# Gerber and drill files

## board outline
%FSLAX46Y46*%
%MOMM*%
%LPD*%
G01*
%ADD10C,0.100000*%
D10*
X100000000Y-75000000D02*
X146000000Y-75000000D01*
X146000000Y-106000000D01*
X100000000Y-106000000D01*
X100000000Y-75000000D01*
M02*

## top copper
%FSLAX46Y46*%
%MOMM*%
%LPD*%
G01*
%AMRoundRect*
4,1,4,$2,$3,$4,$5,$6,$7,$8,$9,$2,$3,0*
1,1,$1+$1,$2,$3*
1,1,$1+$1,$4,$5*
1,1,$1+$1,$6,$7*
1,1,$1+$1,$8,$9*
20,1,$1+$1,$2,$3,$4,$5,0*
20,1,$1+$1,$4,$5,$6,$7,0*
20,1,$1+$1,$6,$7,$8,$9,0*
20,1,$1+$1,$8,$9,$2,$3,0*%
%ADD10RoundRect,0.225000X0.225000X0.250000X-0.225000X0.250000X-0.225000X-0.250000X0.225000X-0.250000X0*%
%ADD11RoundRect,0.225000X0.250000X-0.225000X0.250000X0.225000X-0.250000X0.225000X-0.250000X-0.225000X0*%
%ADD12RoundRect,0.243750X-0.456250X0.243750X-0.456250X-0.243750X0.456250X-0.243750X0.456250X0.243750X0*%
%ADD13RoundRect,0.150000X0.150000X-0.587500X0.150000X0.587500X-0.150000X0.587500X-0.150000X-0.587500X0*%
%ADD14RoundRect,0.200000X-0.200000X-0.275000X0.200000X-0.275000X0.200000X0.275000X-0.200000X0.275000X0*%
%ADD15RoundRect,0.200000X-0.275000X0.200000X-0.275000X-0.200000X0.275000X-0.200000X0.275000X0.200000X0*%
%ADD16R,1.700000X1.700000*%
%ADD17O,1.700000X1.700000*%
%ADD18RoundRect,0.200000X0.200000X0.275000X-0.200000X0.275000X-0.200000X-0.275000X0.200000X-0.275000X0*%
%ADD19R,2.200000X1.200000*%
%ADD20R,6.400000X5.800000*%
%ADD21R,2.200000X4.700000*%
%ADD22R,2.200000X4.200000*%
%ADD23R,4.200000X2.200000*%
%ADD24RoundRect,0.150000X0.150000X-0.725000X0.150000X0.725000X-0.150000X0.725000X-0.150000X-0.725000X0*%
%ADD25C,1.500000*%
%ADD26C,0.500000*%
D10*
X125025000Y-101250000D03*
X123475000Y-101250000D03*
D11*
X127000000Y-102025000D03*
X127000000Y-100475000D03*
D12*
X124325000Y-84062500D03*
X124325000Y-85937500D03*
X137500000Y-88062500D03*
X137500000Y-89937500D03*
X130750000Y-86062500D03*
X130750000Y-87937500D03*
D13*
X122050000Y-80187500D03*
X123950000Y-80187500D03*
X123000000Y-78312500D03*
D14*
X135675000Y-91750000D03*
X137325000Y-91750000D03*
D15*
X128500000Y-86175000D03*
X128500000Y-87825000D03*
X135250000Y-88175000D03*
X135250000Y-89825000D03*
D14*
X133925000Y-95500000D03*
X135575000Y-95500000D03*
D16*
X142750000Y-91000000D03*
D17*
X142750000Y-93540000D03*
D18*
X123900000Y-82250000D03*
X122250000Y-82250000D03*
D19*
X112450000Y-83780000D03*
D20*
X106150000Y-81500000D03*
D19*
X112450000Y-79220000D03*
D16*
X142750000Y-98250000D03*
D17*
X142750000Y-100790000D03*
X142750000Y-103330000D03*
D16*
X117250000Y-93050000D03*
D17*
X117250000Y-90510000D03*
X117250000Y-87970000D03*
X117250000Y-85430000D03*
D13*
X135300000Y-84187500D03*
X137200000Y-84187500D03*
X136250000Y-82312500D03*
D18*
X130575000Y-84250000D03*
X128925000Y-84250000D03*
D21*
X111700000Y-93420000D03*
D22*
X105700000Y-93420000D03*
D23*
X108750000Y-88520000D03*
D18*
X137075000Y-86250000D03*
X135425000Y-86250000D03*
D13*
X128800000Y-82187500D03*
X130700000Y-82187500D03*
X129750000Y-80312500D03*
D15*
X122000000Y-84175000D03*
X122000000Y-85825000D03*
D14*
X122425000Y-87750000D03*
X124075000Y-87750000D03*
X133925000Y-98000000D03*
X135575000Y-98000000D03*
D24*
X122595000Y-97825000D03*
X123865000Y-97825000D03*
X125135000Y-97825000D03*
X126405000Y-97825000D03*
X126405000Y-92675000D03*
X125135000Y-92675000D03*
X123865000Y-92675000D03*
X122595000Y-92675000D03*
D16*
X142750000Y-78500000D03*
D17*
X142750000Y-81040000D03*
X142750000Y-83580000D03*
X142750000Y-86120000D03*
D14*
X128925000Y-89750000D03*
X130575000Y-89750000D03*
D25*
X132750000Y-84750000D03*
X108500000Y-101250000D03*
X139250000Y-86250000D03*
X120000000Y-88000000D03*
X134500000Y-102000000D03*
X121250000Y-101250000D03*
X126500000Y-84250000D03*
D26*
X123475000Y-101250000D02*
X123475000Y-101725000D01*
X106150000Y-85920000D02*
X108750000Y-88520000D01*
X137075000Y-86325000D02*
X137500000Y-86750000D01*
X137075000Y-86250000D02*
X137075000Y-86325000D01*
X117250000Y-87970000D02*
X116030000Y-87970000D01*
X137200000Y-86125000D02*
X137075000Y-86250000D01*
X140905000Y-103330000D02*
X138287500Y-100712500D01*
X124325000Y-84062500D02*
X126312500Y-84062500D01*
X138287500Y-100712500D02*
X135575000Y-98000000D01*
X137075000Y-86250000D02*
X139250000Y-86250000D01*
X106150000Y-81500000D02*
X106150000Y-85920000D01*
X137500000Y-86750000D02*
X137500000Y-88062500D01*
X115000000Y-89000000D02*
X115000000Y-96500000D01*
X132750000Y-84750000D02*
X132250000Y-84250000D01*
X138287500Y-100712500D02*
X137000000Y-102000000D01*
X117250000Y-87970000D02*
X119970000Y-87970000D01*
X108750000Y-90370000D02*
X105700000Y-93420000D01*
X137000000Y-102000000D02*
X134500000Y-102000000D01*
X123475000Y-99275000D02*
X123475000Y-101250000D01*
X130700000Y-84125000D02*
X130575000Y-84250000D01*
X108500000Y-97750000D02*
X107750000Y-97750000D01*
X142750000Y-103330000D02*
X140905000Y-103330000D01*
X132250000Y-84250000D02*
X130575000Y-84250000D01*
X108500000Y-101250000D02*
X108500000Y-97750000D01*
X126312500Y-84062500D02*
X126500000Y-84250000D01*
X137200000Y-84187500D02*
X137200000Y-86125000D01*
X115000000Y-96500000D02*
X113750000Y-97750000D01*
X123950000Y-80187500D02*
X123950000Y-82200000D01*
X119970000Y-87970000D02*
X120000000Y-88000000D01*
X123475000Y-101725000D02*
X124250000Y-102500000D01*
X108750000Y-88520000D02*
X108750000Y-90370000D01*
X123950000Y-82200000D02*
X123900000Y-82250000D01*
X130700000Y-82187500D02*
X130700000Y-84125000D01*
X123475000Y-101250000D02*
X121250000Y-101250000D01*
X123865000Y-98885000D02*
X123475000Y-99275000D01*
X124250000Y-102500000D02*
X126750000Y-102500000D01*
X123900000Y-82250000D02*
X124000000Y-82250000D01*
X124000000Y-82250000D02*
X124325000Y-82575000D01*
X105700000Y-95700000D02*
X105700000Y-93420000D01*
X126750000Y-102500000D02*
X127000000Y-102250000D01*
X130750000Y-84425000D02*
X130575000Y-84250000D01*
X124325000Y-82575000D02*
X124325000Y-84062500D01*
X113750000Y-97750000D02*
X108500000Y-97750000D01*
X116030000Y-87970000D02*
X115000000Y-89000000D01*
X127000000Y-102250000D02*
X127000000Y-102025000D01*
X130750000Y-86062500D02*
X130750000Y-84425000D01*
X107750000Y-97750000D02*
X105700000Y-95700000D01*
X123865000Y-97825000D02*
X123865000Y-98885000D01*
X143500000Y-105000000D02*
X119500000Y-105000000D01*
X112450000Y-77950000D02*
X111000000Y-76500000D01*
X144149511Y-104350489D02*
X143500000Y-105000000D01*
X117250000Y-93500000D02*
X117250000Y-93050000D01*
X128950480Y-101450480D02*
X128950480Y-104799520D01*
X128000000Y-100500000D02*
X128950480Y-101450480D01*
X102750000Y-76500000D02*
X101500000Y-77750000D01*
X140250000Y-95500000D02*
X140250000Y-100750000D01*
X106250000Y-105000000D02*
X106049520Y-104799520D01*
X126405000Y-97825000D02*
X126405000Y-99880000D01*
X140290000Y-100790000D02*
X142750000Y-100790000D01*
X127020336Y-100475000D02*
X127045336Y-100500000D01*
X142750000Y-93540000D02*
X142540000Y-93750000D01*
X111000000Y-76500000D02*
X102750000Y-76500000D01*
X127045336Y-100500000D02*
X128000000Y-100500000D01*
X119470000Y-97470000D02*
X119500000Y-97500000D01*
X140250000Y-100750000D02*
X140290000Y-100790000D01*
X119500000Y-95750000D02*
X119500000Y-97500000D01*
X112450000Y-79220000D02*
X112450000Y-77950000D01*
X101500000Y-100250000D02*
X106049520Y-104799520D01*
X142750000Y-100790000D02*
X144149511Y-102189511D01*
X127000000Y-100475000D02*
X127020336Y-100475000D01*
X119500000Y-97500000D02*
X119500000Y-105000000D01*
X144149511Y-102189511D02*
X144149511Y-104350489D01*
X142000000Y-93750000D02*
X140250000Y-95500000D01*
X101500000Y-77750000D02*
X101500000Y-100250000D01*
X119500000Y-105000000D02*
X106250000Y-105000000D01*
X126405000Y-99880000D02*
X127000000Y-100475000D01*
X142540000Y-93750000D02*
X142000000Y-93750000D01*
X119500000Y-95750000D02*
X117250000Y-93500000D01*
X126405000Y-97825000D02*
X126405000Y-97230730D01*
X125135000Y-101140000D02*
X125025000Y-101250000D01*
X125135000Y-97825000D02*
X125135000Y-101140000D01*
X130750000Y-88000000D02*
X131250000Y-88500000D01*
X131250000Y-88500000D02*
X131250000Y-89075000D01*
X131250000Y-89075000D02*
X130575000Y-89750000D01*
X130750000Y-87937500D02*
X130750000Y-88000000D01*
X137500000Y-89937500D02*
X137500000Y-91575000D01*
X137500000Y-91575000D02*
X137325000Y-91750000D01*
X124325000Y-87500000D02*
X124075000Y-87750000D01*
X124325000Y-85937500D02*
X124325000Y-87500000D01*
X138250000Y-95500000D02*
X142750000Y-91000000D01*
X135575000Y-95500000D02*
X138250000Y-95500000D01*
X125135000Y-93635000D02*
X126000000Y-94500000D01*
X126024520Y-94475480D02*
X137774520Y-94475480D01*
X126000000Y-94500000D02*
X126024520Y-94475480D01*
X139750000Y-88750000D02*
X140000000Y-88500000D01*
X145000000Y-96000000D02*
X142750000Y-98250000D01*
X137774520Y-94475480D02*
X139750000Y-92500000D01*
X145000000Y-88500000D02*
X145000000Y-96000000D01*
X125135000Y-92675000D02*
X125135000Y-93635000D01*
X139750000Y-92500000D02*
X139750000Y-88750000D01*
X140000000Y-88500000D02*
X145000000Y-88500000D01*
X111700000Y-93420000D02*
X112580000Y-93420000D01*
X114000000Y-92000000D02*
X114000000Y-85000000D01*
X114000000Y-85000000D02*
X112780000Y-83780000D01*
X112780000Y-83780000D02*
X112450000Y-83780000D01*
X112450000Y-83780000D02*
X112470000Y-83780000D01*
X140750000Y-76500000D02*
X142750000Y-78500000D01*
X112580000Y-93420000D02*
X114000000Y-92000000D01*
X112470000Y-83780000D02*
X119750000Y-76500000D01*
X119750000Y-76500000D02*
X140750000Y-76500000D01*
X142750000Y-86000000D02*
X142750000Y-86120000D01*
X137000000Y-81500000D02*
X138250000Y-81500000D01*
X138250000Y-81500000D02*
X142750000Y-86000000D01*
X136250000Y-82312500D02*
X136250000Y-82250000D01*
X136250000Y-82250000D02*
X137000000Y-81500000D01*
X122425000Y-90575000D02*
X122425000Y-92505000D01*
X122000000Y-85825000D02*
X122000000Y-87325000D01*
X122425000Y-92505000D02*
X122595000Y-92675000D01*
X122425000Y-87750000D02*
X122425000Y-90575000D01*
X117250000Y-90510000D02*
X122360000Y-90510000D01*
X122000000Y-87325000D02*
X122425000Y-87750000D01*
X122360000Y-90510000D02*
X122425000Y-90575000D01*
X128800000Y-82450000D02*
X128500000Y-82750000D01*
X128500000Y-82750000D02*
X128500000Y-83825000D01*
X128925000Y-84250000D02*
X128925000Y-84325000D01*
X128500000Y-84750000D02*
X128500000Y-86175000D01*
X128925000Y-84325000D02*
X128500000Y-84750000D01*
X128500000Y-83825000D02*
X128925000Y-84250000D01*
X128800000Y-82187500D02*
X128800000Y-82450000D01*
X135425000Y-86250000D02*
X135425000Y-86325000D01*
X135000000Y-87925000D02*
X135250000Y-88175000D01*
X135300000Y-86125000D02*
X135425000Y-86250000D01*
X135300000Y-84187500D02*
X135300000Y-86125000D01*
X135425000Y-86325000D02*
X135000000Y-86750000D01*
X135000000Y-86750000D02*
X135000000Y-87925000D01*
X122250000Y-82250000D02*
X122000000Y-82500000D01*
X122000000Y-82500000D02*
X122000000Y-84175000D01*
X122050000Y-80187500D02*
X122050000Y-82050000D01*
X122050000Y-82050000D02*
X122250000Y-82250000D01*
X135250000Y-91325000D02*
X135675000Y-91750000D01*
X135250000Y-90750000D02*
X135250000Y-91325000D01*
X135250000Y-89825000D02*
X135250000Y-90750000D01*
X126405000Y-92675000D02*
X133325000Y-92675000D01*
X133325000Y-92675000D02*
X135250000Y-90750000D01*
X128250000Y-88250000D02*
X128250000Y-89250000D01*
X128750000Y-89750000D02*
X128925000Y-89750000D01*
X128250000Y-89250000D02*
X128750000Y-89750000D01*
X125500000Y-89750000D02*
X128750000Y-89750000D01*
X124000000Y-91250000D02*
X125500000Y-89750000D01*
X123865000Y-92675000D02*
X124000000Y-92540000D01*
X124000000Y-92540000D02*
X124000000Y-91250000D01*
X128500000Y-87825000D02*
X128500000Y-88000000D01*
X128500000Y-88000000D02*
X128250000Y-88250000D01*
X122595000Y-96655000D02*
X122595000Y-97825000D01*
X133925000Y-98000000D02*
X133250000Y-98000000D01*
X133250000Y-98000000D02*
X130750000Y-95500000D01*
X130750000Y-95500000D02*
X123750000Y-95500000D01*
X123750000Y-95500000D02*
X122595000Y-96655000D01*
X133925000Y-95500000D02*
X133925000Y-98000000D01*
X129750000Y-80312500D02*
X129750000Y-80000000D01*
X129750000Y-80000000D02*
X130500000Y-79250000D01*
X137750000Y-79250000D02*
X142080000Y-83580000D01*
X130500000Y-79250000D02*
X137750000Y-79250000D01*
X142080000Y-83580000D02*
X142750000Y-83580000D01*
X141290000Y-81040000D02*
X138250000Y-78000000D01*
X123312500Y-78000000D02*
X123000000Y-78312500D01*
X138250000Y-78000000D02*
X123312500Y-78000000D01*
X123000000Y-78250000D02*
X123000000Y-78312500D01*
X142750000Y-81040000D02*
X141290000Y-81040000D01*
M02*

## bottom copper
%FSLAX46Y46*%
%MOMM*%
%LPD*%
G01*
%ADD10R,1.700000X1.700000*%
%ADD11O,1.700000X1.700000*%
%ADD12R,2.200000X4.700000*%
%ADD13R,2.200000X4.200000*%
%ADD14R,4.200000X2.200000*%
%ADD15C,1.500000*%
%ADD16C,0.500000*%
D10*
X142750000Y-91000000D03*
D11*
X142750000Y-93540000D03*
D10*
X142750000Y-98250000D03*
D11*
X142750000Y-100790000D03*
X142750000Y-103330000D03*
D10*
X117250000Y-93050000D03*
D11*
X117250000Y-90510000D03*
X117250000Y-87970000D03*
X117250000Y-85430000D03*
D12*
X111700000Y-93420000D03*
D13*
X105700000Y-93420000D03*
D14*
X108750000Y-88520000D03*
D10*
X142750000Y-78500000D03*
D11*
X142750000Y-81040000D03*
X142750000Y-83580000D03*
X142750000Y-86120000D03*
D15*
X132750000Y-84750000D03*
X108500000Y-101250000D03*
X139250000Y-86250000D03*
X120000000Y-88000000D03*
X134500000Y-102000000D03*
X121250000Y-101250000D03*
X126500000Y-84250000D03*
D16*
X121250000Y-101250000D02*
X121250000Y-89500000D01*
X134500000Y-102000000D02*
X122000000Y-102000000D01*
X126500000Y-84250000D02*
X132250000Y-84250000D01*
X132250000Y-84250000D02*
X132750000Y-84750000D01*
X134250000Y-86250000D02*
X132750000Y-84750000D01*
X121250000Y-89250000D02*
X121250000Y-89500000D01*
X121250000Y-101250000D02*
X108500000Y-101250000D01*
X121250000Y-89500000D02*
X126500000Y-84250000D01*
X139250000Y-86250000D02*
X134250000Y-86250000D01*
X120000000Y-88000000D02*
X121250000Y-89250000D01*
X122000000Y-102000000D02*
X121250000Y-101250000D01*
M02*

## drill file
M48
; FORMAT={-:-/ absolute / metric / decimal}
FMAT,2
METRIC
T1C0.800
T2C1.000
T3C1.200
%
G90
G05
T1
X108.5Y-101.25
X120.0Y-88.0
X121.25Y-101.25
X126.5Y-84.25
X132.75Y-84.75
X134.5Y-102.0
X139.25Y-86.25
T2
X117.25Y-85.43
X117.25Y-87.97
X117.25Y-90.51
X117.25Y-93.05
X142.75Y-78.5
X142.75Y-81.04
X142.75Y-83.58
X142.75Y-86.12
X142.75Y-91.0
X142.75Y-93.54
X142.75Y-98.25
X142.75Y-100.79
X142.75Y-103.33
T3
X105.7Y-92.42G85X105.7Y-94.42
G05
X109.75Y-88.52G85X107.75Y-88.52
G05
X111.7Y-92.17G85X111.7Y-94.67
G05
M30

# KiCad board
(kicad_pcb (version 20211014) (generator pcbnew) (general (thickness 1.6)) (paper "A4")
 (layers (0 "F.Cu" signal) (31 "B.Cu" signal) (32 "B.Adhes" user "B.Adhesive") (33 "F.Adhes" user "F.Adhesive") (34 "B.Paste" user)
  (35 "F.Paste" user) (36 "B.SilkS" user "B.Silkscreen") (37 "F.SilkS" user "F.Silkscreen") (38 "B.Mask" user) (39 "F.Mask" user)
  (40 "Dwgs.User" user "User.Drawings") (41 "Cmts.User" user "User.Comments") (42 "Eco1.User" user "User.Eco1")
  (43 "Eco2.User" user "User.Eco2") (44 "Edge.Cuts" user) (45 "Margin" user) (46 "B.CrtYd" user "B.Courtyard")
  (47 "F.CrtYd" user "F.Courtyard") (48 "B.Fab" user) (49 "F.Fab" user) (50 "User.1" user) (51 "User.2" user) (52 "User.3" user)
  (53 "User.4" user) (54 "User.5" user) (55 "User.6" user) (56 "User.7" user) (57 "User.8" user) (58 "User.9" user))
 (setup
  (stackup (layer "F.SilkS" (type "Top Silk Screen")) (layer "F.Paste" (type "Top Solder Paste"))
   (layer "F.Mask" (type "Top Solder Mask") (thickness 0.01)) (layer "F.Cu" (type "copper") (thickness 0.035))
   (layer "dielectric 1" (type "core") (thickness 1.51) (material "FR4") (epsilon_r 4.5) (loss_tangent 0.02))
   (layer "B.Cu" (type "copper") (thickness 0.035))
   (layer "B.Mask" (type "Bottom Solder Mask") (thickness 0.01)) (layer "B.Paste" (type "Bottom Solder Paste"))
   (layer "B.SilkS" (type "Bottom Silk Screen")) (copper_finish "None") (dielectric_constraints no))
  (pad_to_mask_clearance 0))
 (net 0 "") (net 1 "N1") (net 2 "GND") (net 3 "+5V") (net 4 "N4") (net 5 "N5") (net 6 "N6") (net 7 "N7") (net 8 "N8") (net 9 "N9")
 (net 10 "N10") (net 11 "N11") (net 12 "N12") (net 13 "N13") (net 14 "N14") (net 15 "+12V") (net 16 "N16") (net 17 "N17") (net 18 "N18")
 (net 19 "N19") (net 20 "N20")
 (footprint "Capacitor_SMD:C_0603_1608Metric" (layer "F.Cu") (at 124.25 101.25 180)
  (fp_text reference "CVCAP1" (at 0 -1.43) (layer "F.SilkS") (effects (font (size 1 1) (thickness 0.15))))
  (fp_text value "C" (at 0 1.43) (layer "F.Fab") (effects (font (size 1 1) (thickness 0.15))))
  (pad "1" smd roundrect (at -0.775 0 180) (size 0.9 0.95) (layers "F.Cu" "F.Paste" "F.Mask") (roundrect_rratio 0.25) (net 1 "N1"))
  (pad "2" smd roundrect (at 0.775 0 180) (size 0.9 0.95) (layers "F.Cu" "F.Paste" "F.Mask") (roundrect_rratio 0.25) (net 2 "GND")))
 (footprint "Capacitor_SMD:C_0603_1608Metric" (layer "F.Cu") (at 127 101.25 90)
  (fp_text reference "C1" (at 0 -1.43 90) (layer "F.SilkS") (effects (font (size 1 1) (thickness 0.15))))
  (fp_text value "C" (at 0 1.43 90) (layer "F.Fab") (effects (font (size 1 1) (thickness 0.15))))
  (pad "1" smd roundrect (at -0.775 0 90) (size 0.9 0.95) (layers "F.Cu" "F.Paste" "F.Mask") (roundrect_rratio 0.25) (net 2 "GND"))
  (pad "2" smd roundrect (at 0.775 0 90) (size 0.9 0.95) (layers "F.Cu" "F.Paste" "F.Mask") (roundrect_rratio 0.25) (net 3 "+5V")))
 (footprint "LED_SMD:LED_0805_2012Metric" (layer "F.Cu") (at 124.325 85 -90)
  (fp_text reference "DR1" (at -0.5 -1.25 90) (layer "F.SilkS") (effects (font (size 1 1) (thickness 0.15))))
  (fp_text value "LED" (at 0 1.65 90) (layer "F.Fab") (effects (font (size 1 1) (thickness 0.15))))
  (pad "1" smd roundrect (at -0.9375 0 270) (size 0.975 1.4) (layers "F.Cu" "F.Paste" "F.Mask") (roundrect_rratio 0.25) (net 2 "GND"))
  (pad "2" smd roundrect (at 0.9375 0 270) (size 0.975 1.4) (layers "F.Cu" "F.Paste" "F.Mask") (roundrect_rratio 0.25) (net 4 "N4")))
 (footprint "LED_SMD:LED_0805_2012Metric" (layer "F.Cu") (at 137.5 89 -90)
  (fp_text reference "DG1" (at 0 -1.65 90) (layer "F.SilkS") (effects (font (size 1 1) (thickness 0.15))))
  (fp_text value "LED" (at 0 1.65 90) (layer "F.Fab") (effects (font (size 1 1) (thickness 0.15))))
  (pad "1" smd roundrect (at -0.9375 0 270) (size 0.975 1.4) (layers "F.Cu" "F.Paste" "F.Mask") (roundrect_rratio 0.25) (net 2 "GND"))
  (pad "2" smd roundrect (at 0.9375 0 270) (size 0.975 1.4) (layers "F.Cu" "F.Paste" "F.Mask") (roundrect_rratio 0.25) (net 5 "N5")))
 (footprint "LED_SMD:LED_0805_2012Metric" (layer "F.Cu") (at 130.75 87 -90)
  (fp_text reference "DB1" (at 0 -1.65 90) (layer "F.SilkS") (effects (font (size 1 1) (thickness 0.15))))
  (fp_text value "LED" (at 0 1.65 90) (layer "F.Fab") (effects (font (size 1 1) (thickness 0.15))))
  (pad "1" smd roundrect (at -0.9375 0 270) (size 0.975 1.4) (layers "F.Cu" "F.Paste" "F.Mask") (roundrect_rratio 0.25) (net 2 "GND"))
  (pad "2" smd roundrect (at 0.9375 0 270) (size 0.975 1.4) (layers "F.Cu" "F.Paste" "F.Mask") (roundrect_rratio 0.25) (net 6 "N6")))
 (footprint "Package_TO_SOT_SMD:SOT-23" (layer "F.Cu") (at 123 79.25 90)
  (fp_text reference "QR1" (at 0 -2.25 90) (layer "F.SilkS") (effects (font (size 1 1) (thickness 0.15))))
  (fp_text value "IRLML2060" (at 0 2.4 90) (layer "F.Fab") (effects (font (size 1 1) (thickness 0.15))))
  (pad "1" smd roundrect (at -0.9375 -0.95 90) (size 1.475 0.6) (layers "F.Cu" "F.Paste" "F.Mask") (roundrect_rratio 0.25) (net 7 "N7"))
  (pad "2" smd roundrect (at -0.9375 0.95 90) (size 1.475 0.6) (layers "F.Cu" "F.Paste" "F.Mask") (roundrect_rratio 0.25) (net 2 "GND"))
  (pad "3" smd roundrect (at 0.9375 0 90) (size 1.475 0.6) (layers "F.Cu" "F.Paste" "F.Mask") (roundrect_rratio 0.25) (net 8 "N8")))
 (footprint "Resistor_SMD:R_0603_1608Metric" (layer "F.Cu") (at 136.5 91.75)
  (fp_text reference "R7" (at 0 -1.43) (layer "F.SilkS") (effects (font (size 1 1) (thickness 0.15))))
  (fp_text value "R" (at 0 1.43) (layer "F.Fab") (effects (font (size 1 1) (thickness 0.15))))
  (pad "1" smd roundrect (at -0.825 0) (size 0.8 0.95) (layers "F.Cu" "F.Paste" "F.Mask") (roundrect_rratio 0.25) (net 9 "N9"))
  (pad "2" smd roundrect (at 0.825 0) (size 0.8 0.95) (layers "F.Cu" "F.Paste" "F.Mask") (roundrect_rratio 0.25) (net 5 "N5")))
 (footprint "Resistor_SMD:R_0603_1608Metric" (layer "F.Cu") (at 128.5 87 -90)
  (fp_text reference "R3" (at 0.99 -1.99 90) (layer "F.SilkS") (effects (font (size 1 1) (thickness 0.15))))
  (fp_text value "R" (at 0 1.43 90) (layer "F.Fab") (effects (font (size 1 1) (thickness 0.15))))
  (pad "1" smd roundrect (at -0.825 0 270) (size 0.8 0.95) (layers "F.Cu" "F.Paste" "F.Mask") (roundrect_rratio 0.25) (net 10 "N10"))
  (pad "2" smd roundrect (at 0.825 0 270) (size 0.8 0.95) (layers "F.Cu" "F.Paste" "F.Mask") (roundrect_rratio 0.25) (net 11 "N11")))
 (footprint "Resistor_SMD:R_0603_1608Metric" (layer "F.Cu") (at 135.25 89 -90)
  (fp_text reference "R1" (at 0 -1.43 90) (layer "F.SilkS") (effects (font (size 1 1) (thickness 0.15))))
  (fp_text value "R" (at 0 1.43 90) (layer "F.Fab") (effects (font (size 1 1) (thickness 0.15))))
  (pad "1" smd roundrect (at -0.825 0 270) (size 0.8 0.95) (layers "F.Cu" "F.Paste" "F.Mask") (roundrect_rratio 0.25) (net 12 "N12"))
  (pad "2" smd roundrect (at 0.825 0 270) (size 0.8 0.95) (layers "F.Cu" "F.Paste" "F.Mask") (roundrect_rratio 0.25) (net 9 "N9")))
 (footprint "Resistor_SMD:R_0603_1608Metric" (layer "F.Cu") (at 134.75 95.5)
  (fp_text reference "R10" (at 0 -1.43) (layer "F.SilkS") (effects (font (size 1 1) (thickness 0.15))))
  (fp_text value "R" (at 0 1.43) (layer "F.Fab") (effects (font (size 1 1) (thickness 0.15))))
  (pad "1" smd roundrect (at -0.825 0) (size 0.8 0.95) (layers "F.Cu" "F.Paste" "F.Mask") (roundrect_rratio 0.25) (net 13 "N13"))
  (pad "2" smd roundrect (at 0.825 0) (size 0.8 0.95) (layers "F.Cu" "F.Paste" "F.Mask") (roundrect_rratio 0.25) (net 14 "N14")))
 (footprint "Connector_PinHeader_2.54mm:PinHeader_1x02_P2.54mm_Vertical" (layer "F.Cu") (at 142.75 91)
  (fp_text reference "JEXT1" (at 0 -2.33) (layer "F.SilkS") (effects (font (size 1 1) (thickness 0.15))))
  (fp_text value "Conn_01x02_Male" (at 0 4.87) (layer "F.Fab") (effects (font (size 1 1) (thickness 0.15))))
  (pad "1" thru_hole rect (at 0 0) (size 1.7 1.7) (drill 1) (layers *.Cu *.Mask) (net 14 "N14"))
  (pad "2" thru_hole oval (at 0 2.54) (size 1.7 1.7) (drill 1) (layers *.Cu *.Mask) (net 3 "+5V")))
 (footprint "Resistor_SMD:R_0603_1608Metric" (layer "F.Cu") (at 123.075 82.25 180)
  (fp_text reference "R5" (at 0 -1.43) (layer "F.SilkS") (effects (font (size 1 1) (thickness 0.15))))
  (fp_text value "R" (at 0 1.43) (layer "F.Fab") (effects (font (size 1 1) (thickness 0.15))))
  (pad "1" smd roundrect (at -0.825 0 180) (size 0.8 0.95) (layers "F.Cu" "F.Paste" "F.Mask") (roundrect_rratio 0.25) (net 2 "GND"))
  (pad "2" smd roundrect (at 0.825 0 180) (size 0.8 0.95) (layers "F.Cu" "F.Paste" "F.Mask") (roundrect_rratio 0.25) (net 7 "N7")))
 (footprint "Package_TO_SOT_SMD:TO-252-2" (layer "F.Cu") (at 108.25 81.5 180)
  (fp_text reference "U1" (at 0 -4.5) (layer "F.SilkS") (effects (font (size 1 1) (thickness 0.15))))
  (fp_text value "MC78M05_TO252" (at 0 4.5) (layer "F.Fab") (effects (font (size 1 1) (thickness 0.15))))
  (pad "" smd rect (at 3.775 1.525 180) (size 3.05 2.75) (layers "F.Paste"))
  (pad "" smd rect (at 0.425 -1.525 180) (size 3.05 2.75) (layers "F.Paste"))
  (pad "" smd rect (at 0.425 1.525 180) (size 3.05 2.75) (layers "F.Paste"))
  (pad "" smd rect (at 3.775 -1.525 180) (size 3.05 2.75) (layers "F.Paste"))
  (pad "1" smd rect (at -4.2 -2.28 180) (size 2.2 1.2) (layers "F.Cu" "F.Paste" "F.Mask") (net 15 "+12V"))
  (pad "2" smd rect (at 2.1 0 180) (size 6.4 5.8) (layers "F.Cu" "F.Mask") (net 2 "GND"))
  (pad "3" smd rect (at -4.2 2.28 180) (size 2.2 1.2) (layers "F.Cu" "F.Paste" "F.Mask") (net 3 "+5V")))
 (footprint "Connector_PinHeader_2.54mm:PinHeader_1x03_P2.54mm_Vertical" (layer "F.Cu") (at 142.75 98.25)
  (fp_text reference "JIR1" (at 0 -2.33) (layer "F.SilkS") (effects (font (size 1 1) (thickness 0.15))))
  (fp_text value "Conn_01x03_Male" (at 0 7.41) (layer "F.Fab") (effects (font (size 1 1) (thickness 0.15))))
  (pad "1" thru_hole rect (at 0 0) (size 1.7 1.7) (drill 1) (layers *.Cu *.Mask) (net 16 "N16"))
  (pad "2" thru_hole oval (at 0 2.54) (size 1.7 1.7) (drill 1) (layers *.Cu *.Mask) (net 3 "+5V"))
  (pad "3" thru_hole oval (at 0 5.08) (size 1.7 1.7) (drill 1) (layers *.Cu *.Mask) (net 2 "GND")))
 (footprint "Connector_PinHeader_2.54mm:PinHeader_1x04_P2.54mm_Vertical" (layer "F.Cu") (at 117.25 93.05 180)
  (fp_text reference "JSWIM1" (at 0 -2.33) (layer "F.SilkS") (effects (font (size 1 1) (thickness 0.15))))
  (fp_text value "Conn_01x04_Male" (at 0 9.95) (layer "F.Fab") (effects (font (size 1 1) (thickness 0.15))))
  (pad "1" thru_hole rect (at 0 0 180) (size 1.7 1.7) (drill 1) (layers *.Cu *.Mask) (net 3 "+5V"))
  (pad "2" thru_hole oval (at 0 2.54 180) (size 1.7 1.7) (drill 1) (layers *.Cu *.Mask) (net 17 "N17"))
  (pad "3" thru_hole oval (at 0 5.08 180) (size 1.7 1.7) (drill 1) (layers *.Cu *.Mask) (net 2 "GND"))
  (pad "4" thru_hole oval (at 0 7.62 180) (size 1.7 1.7) (drill 1) (layers *.Cu *.Mask) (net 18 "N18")))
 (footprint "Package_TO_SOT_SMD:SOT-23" (layer "F.Cu") (at 136.25 83.25 90)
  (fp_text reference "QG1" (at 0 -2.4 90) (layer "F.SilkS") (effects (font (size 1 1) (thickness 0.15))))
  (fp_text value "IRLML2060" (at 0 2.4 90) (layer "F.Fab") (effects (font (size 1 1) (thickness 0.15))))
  (pad "1" smd roundrect (at -0.9375 -0.95 90) (size 1.475 0.6) (layers "F.Cu" "F.Paste" "F.Mask") (roundrect_rratio 0.25) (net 12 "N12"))
  (pad "2" smd roundrect (at -0.9375 0.95 90) (size 1.475 0.6) (layers "F.Cu" "F.Paste" "F.Mask") (roundrect_rratio 0.25) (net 2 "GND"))
  (pad "3" smd roundrect (at 0.9375 0 90) (size 1.475 0.6) (layers "F.Cu" "F.Paste" "F.Mask") (roundrect_rratio 0.25) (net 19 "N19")))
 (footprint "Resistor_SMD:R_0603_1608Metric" (layer "F.Cu") (at 129.75 84.25 180)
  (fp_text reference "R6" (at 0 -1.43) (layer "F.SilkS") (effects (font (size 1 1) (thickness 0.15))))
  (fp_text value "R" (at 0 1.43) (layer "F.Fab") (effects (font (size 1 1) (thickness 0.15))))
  (pad "1" smd roundrect (at -0.825 0 180) (size 0.8 0.95) (layers "F.Cu" "F.Paste" "F.Mask") (roundrect_rratio 0.25) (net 2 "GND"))
  (pad "2" smd roundrect (at 0.825 0 180) (size 0.8 0.95) (layers "F.Cu" "F.Paste" "F.Mask") (roundrect_rratio 0.25) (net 10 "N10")))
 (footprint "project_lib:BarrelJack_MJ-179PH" (layer "F.Cu") (at 112.5 94 -90)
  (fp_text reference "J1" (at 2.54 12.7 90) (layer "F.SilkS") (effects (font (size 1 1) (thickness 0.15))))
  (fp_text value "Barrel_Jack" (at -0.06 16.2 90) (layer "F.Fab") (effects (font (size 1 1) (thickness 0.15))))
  (pad "1" thru_hole rect (at -0.58 0.8 270) (size 4.7 2.2) (drill oval 3.7 1.2) (layers *.Cu *.Mask) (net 15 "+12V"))
  (pad "2" thru_hole rect (at -0.58 6.8 270) (size 4.2 2.2) (drill oval 3.2 1.2) (layers *.Cu *.Mask) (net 2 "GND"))
  (pad "3" thru_hole rect (at -5.48 3.75 270) (size 2.2 4.2) (drill oval 1.2 3.2) (layers *.Cu *.Mask) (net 2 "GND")))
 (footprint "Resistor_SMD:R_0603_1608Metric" (layer "F.Cu") (at 136.25 86.25 180)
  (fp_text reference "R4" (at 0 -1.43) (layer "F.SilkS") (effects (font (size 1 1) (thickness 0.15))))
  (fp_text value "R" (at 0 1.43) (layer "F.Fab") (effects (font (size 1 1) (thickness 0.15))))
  (pad "1" smd roundrect (at -0.825 0 180) (size 0.8 0.95) (layers "F.Cu" "F.Paste" "F.Mask") (roundrect_rratio 0.25) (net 2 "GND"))
  (pad "2" smd roundrect (at 0.825 0 180) (size 0.8 0.95) (layers "F.Cu" "F.Paste" "F.Mask") (roundrect_rratio 0.25) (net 12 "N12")))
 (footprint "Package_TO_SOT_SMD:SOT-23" (layer "F.Cu") (at 129.75 81.25 90)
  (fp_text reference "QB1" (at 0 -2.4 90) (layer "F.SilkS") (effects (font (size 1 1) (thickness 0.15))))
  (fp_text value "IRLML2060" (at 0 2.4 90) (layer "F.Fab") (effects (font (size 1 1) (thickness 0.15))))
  (pad "1" smd roundrect (at -0.9375 -0.95 90) (size 1.475 0.6) (layers "F.Cu" "F.Paste" "F.Mask") (roundrect_rratio 0.25) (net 10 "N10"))
  (pad "2" smd roundrect (at -0.9375 0.95 90) (size 1.475 0.6) (layers "F.Cu" "F.Paste" "F.Mask") (roundrect_rratio 0.25) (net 2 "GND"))
  (pad "3" smd roundrect (at 0.9375 0 90) (size 1.475 0.6) (layers "F.Cu" "F.Paste" "F.Mask") (roundrect_rratio 0.25) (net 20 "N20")))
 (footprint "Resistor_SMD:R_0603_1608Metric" (layer "F.Cu") (at 122 85 -90)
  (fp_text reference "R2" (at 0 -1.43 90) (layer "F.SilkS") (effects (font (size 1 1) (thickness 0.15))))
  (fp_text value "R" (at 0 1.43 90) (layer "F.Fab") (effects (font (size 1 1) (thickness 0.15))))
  (pad "1" smd roundrect (at -0.825 0 270) (size 0.8 0.95) (layers "F.Cu" "F.Paste" "F.Mask") (roundrect_rratio 0.25) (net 7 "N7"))
  (pad "2" smd roundrect (at 0.825 0 270) (size 0.8 0.95) (layers "F.Cu" "F.Paste" "F.Mask") (roundrect_rratio 0.25) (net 17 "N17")))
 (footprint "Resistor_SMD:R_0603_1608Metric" (layer "F.Cu") (at 123.25 87.75)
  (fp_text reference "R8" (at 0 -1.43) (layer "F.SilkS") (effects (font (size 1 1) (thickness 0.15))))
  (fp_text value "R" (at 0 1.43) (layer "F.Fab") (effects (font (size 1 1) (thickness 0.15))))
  (pad "1" smd roundrect (at -0.825 0) (size 0.8 0.95) (layers "F.Cu" "F.Paste" "F.Mask") (roundrect_rratio 0.25) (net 17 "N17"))
  (pad "2" smd roundrect (at 0.825 0) (size 0.8 0.95) (layers "F.Cu" "F.Paste" "F.Mask") (roundrect_rratio 0.25) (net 4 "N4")))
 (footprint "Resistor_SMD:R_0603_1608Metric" (layer "F.Cu") (at 134.75 98)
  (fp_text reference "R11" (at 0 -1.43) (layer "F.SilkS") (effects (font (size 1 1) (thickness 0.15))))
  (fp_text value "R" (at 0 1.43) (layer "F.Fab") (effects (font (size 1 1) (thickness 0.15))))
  (pad "1" smd roundrect (at -0.825 0) (size 0.8 0.95) (layers "F.Cu" "F.Paste" "F.Mask") (roundrect_rratio 0.25) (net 13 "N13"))
  (pad "2" smd roundrect (at 0.825 0) (size 0.8 0.95) (layers "F.Cu" "F.Paste" "F.Mask") (roundrect_rratio 0.25) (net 2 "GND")))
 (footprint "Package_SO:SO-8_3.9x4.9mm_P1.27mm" (layer "F.Cu") (at 124.5 95.25 90)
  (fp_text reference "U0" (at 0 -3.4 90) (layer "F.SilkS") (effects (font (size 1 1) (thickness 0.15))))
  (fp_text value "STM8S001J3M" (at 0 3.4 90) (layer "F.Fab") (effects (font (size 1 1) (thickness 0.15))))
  (pad "1" smd roundrect (at -2.575 -1.905 90) (size 1.75 0.6) (layers "F.Cu" "F.Paste" "F.Mask") (roundrect_rratio 0.25) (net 13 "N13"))
  (pad "2" smd roundrect (at -2.575 -0.635 90) (size 1.75 0.6) (layers "F.Cu" "F.Paste" "F.Mask") (roundrect_rratio 0.25) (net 2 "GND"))
  (pad "3" smd roundrect (at -2.575 0.635 90) (size 1.75 0.6) (layers "F.Cu" "F.Paste" "F.Mask") (roundrect_rratio 0.25) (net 1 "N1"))
  (pad "4" smd roundrect (at -2.575 1.905 90) (size 1.75 0.6) (layers "F.Cu" "F.Paste" "F.Mask") (roundrect_rratio 0.25) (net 3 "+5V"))
  (pad "5" smd roundrect (at 2.575 1.905 90) (size 1.75 0.6) (layers "F.Cu" "F.Paste" "F.Mask") (roundrect_rratio 0.25) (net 9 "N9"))
  (pad "6" smd roundrect (at 2.575 0.635 90) (size 1.75 0.6) (layers "F.Cu" "F.Paste" "F.Mask") (roundrect_rratio 0.25) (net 16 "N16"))
  (pad "7" smd roundrect (at 2.575 -0.635 90) (size 1.75 0.6) (layers "F.Cu" "F.Paste" "F.Mask") (roundrect_rratio 0.25) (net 11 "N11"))
  (pad "8" smd roundrect (at 2.575 -1.905 90) (size 1.75 0.6) (layers "F.Cu" "F.Paste" "F.Mask") (roundrect_rratio 0.25) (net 17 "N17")))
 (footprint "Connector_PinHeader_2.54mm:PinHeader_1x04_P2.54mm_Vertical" (layer "F.Cu") (at 142.75 78.5)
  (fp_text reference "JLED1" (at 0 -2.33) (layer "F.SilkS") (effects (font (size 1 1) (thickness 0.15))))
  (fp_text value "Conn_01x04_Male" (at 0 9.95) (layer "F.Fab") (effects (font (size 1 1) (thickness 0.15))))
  (pad "1" thru_hole rect (at 0 0) (size 1.7 1.7) (drill 1) (layers *.Cu *.Mask) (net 15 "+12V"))
  (pad "2" thru_hole oval (at 0 2.54) (size 1.7 1.7) (drill 1) (layers *.Cu *.Mask) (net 8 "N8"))
  (pad "3" thru_hole oval (at 0 5.08) (size 1.7 1.7) (drill 1) (layers *.Cu *.Mask) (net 20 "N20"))
  (pad "4" thru_hole oval (at 0 7.62) (size 1.7 1.7) (drill 1) (layers *.Cu *.Mask) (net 19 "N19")))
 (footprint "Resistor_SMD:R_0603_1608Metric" (layer "F.Cu") (at 129.75 89.75)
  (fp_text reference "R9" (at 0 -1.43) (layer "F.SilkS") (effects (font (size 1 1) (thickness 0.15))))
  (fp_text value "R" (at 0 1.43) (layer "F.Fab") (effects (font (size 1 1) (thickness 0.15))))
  (pad "1" smd roundrect (at -0.825 0) (size 0.8 0.95) (layers "F.Cu" "F.Paste" "F.Mask") (roundrect_rratio 0.25) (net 11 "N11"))
  (pad "2" smd roundrect (at 0.825 0) (size 0.8 0.95) (layers "F.Cu" "F.Paste" "F.Mask") (roundrect_rratio 0.25) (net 6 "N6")))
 (gr_rect (start 100 75) (end 146 106) (layer "Edge.Cuts") (width 0.1) (fill none))
 (segment (start 123.475 101.25) (end 123.475 101.725) (width 0.5) (layer "F.Cu") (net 2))
 (segment (start 106.15 85.92) (end 108.75 88.52) (width 0.5) (layer "F.Cu") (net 2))
 (segment (start 137.075 86.325) (end 137.5 86.75) (width 0.5) (layer "F.Cu") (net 2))
 (segment (start 137.075 86.25) (end 137.075 86.325) (width 0.5) (layer "F.Cu") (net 2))
 (segment (start 117.25 87.97) (end 116.03 87.97) (width 0.5) (layer "F.Cu") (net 2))
 (segment (start 137.2 86.125) (end 137.075 86.25) (width 0.5) (layer "F.Cu") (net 2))
 (segment (start 140.905 103.33) (end 138.2875 100.7125) (width 0.5) (layer "F.Cu") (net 2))
 (segment (start 124.325 84.0625) (end 126.3125 84.0625) (width 0.5) (layer "F.Cu") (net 2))
 (segment (start 138.2875 100.7125) (end 135.575 98) (width 0.5) (layer "F.Cu") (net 2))
 (segment (start 137.075 86.25) (end 139.25 86.25) (width 0.5) (layer "F.Cu") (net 2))
 (segment (start 106.15 81.5) (end 106.15 85.92) (width 0.5) (layer "F.Cu") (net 2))
 (segment (start 137.5 86.75) (end 137.5 88.0625) (width 0.5) (layer "F.Cu") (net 2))
 (segment (start 115 89) (end 115 96.5) (width 0.5) (layer "F.Cu") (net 2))
 (segment (start 132.75 84.75) (end 132.25 84.25) (width 0.5) (layer "F.Cu") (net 2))
 (segment (start 138.2875 100.7125) (end 137 102) (width 0.5) (layer "F.Cu") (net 2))
 (segment (start 117.25 87.97) (end 119.97 87.97) (width 0.5) (layer "F.Cu") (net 2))
 (segment (start 108.75 90.37) (end 105.7 93.42) (width 0.5) (layer "F.Cu") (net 2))
 (segment (start 137 102) (end 134.5 102) (width 0.5) (layer "F.Cu") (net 2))
 (segment (start 123.475 99.275) (end 123.475 101.25) (width 0.5) (layer "F.Cu") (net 2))
 (segment (start 130.7 84.125) (end 130.575 84.25) (width 0.5) (layer "F.Cu") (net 2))
 (segment (start 108.5 97.75) (end 107.75 97.75) (width 0.5) (layer "F.Cu") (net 2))
 (segment (start 142.75 103.33) (end 140.905 103.33) (width 0.5) (layer "F.Cu") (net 2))
 (segment (start 132.25 84.25) (end 130.575 84.25) (width 0.5) (layer "F.Cu") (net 2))
 (segment (start 108.5 101.25) (end 108.5 97.75) (width 0.5) (layer "F.Cu") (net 2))
 (segment (start 126.3125 84.0625) (end 126.5 84.25) (width 0.5) (layer "F.Cu") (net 2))
 (segment (start 137.2 84.1875) (end 137.2 86.125) (width 0.5) (layer "F.Cu") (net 2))
 (segment (start 115 96.5) (end 113.75 97.75) (width 0.5) (layer "F.Cu") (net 2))
 (segment (start 123.95 80.1875) (end 123.95 82.2) (width 0.5) (layer "F.Cu") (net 2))
 (segment (start 119.97 87.97) (end 120 88) (width 0.5) (layer "F.Cu") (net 2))
 (segment (start 123.475 101.725) (end 124.25 102.5) (width 0.5) (layer "F.Cu") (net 2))
 (segment (start 108.75 88.52) (end 108.75 90.37) (width 0.5) (layer "F.Cu") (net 2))
 (segment (start 123.95 82.2) (end 123.9 82.25) (width 0.5) (layer "F.Cu") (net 2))
 (segment (start 130.7 82.1875) (end 130.7 84.125) (width 0.5) (layer "F.Cu") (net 2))
 (segment (start 123.475 101.25) (end 121.25 101.25) (width 0.5) (layer "F.Cu") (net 2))
 (segment (start 123.865 98.885) (end 123.475 99.275) (width 0.5) (layer "F.Cu") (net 2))
 (segment (start 124.25 102.5) (end 126.75 102.5) (width 0.5) (layer "F.Cu") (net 2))
 (segment (start 123.9 82.25) (end 124 82.25) (width 0.5) (layer "F.Cu") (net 2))
 (segment (start 124 82.25) (end 124.325 82.575) (width 0.5) (layer "F.Cu") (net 2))
 (segment (start 105.7 95.7) (end 105.7 93.42) (width 0.5) (layer "F.Cu") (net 2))
 (segment (start 126.75 102.5) (end 127 102.25) (width 0.5) (layer "F.Cu") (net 2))
 (segment (start 130.75 84.425) (end 130.575 84.25) (width 0.5) (layer "F.Cu") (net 2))
 (segment (start 124.325 82.575) (end 124.325 84.0625) (width 0.5) (layer "F.Cu") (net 2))
 (segment (start 113.75 97.75) (end 108.5 97.75) (width 0.5) (layer "F.Cu") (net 2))
 (segment (start 116.03 87.97) (end 115 89) (width 0.5) (layer "F.Cu") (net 2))
 (segment (start 127 102.25) (end 127 102.025) (width 0.5) (layer "F.Cu") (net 2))
 (segment (start 130.75 86.0625) (end 130.75 84.425) (width 0.5) (layer "F.Cu") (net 2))
 (segment (start 107.75 97.75) (end 105.7 95.7) (width 0.5) (layer "F.Cu") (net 2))
 (segment (start 123.865 97.825) (end 123.865 98.885) (width 0.5) (layer "F.Cu") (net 2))
 (via (at 132.75 84.75) (size 1.5) (drill 0.8) (layers "F.Cu" "B.Cu") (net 2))
 (via (at 108.5 101.25) (size 1.5) (drill 0.8) (layers "F.Cu" "B.Cu") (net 2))
 (via (at 139.25 86.25) (size 1.5) (drill 0.8) (layers "F.Cu" "B.Cu") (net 2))
 (via (at 120 88) (size 1.5) (drill 0.8) (layers "F.Cu" "B.Cu") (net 2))
 (via (at 134.5 102) (size 1.5) (drill 0.8) (layers "F.Cu" "B.Cu") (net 2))
 (via (at 121.25 101.25) (size 1.5) (drill 0.8) (layers "F.Cu" "B.Cu") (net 2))
 (via (at 126.5 84.25) (size 1.5) (drill 0.8) (layers "F.Cu" "B.Cu") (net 2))
 (segment (start 121.25 101.25) (end 121.25 89.5) (width 0.5) (layer "B.Cu") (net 2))
 (segment (start 134.5 102) (end 122 102) (width 0.5) (layer "B.Cu") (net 2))
 (segment (start 126.5 84.25) (end 132.25 84.25) (width 0.5) (layer "B.Cu") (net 2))
 (segment (start 132.25 84.25) (end 132.75 84.75) (width 0.5) (layer "B.Cu") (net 2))
 (segment (start 134.25 86.25) (end 132.75 84.75) (width 0.5) (layer "B.Cu") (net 2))
 (segment (start 121.25 89.25) (end 121.25 89.5) (width 0.5) (layer "B.Cu") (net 2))
 (segment (start 121.25 101.25) (end 108.5 101.25) (width 0.5) (layer "B.Cu") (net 2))
 (segment (start 121.25 89.5) (end 126.5 84.25) (width 0.5) (layer "B.Cu") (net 2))
 (segment (start 139.25 86.25) (end 134.25 86.25) (width 0.5) (layer "B.Cu") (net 2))
 (segment (start 120 88) (end 121.25 89.25) (width 0.5) (layer "B.Cu") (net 2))
 (segment (start 122 102) (end 121.25 101.25) (width 0.5) (layer "B.Cu") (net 2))
 (segment (start 143.5 105) (end 119.5 105) (width 0.5) (layer "F.Cu") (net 3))
 (segment (start 112.45 77.95) (end 111 76.5) (width 0.5) (layer "F.Cu") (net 3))
 (segment (start 144.149511 104.350489) (end 143.5 105) (width 0.5) (layer "F.Cu") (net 3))
 (segment (start 117.25 93.5) (end 117.25 93.05) (width 0.5) (layer "F.Cu") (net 3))
 (segment (start 128.95048 101.45048) (end 128.95048 104.79952) (width 0.5) (layer "F.Cu") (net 3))
 (segment (start 128 100.5) (end 128.95048 101.45048) (width 0.5) (layer "F.Cu") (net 3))
 (segment (start 102.75 76.5) (end 101.5 77.75) (width 0.5) (layer "F.Cu") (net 3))
 (segment (start 140.25 95.5) (end 140.25 100.75) (width 0.5) (layer "F.Cu") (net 3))
 (segment (start 106.25 105) (end 106.04952 104.79952) (width 0.5) (layer "F.Cu") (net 3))
 (segment (start 126.405 97.825) (end 126.405 99.88) (width 0.5) (layer "F.Cu") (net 3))
 (segment (start 140.29 100.79) (end 142.75 100.79) (width 0.5) (layer "F.Cu") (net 3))
 (segment (start 127.020336 100.475) (end 127.045336 100.5) (width 0.5) (layer "F.Cu") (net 3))
 (segment (start 142.75 93.54) (end 142.54 93.75) (width 0.5) (layer "F.Cu") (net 3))
 (segment (start 111 76.5) (end 102.75 76.5) (width 0.5) (layer "F.Cu") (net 3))
 (segment (start 127.045336 100.5) (end 128 100.5) (width 0.5) (layer "F.Cu") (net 3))
 (segment (start 119.47 97.47) (end 119.5 97.5) (width 0.5) (layer "F.Cu") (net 3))
 (segment (start 140.25 100.75) (end 140.29 100.79) (width 0.5) (layer "F.Cu") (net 3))
 (segment (start 119.5 95.75) (end 119.5 97.5) (width 0.5) (layer "F.Cu") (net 3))
 (segment (start 112.45 79.22) (end 112.45 77.95) (width 0.5) (layer "F.Cu") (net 3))
 (segment (start 101.5 100.25) (end 106.04952 104.79952) (width 0.5) (layer "F.Cu") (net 3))
 (segment (start 142.75 100.79) (end 144.149511 102.189511) (width 0.5) (layer "F.Cu") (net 3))
 (segment (start 127 100.475) (end 127.020336 100.475) (width 0.5) (layer "F.Cu") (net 3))
 (segment (start 119.5 97.5) (end 119.5 105) (width 0.5) (layer "F.Cu") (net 3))
 (segment (start 144.149511 102.189511) (end 144.149511 104.350489) (width 0.5) (layer "F.Cu") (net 3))
 (segment (start 142 93.75) (end 140.25 95.5) (width 0.5) (layer "F.Cu") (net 3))
 (segment (start 101.5 77.75) (end 101.5 100.25) (width 0.5) (layer "F.Cu") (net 3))
 (segment (start 119.5 105) (end 106.25 105) (width 0.5) (layer "F.Cu") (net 3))
 (segment (start 126.405 99.88) (end 127 100.475) (width 0.5) (layer "F.Cu") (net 3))
 (segment (start 142.54 93.75) (end 142 93.75) (width 0.5) (layer "F.Cu") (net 3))
 (segment (start 119.5 95.75) (end 117.25 93.5) (width 0.5) (layer "F.Cu") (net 3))
 (segment (start 126.405 97.825) (end 126.405 97.23073) (width 0.5) (layer "F.Cu") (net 3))
 (segment (start 125.135 101.14) (end 125.025 101.25) (width 0.5) (layer "F.Cu") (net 1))
 (segment (start 125.135 97.825) (end 125.135 101.14) (width 0.5) (layer "F.Cu") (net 1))
 (segment (start 130.75 88) (end 131.25 88.5) (width 0.5) (layer "F.Cu") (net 6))
 (segment (start 131.25 88.5) (end 131.25 89.075) (width 0.5) (layer "F.Cu") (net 6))
 (segment (start 131.25 89.075) (end 130.575 89.75) (width 0.5) (layer "F.Cu") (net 6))
 (segment (start 130.75 87.9375) (end 130.75 88) (width 0.5) (layer "F.Cu") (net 6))
 (segment (start 137.5 89.9375) (end 137.5 91.575) (width 0.5) (layer "F.Cu") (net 5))
 (segment (start 137.5 91.575) (end 137.325 91.75) (width 0.5) (layer "F.Cu") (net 5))
 (segment (start 124.325 87.5) (end 124.075 87.75) (width 0.5) (layer "F.Cu") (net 4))
 (segment (start 124.325 85.9375) (end 124.325 87.5) (width 0.5) (layer "F.Cu") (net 4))
 (segment (start 138.25 95.5) (end 142.75 91) (width 0.5) (layer "F.Cu") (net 14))
 (segment (start 135.575 95.5) (end 138.25 95.5) (width 0.5) (layer "F.Cu") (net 14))
 (segment (start 125.135 93.635) (end 126 94.5) (width 0.5) (layer "F.Cu") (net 16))
 (segment (start 126.02452 94.47548) (end 137.77452 94.47548) (width 0.5) (layer "F.Cu") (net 16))
 (segment (start 126 94.5) (end 126.02452 94.47548) (width 0.5) (layer "F.Cu") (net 16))
 (segment (start 139.75 88.75) (end 140 88.5) (width 0.5) (layer "F.Cu") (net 16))
 (segment (start 145 96) (end 142.75 98.25) (width 0.5) (layer "F.Cu") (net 16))
 (segment (start 137.77452 94.47548) (end 139.75 92.5) (width 0.5) (layer "F.Cu") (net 16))
 (segment (start 145 88.5) (end 145 96) (width 0.5) (layer "F.Cu") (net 16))
 (segment (start 125.135 92.675) (end 125.135 93.635) (width 0.5) (layer "F.Cu") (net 16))
 (segment (start 139.75 92.5) (end 139.75 88.75) (width 0.5) (layer "F.Cu") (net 16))
 (segment (start 140 88.5) (end 145 88.5) (width 0.5) (layer "F.Cu") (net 16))
 (segment (start 111.7 93.42) (end 112.58 93.42) (width 0.5) (layer "F.Cu") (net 15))
 (segment (start 114 92) (end 114 85) (width 0.5) (layer "F.Cu") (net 15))
 (segment (start 114 85) (end 112.78 83.78) (width 0.5) (layer "F.Cu") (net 15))
 (segment (start 112.78 83.78) (end 112.45 83.78) (width 0.5) (layer "F.Cu") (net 15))
 (segment (start 112.45 83.78) (end 112.47 83.78) (width 0.5) (layer "F.Cu") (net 15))
 (segment (start 140.75 76.5) (end 142.75 78.5) (width 0.5) (layer "F.Cu") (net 15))
 (segment (start 112.58 93.42) (end 114 92) (width 0.5) (layer "F.Cu") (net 15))
 (segment (start 112.47 83.78) (end 119.75 76.5) (width 0.5) (layer "F.Cu") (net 15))
 (segment (start 119.75 76.5) (end 140.75 76.5) (width 0.5) (layer "F.Cu") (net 15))
 (segment (start 142.75 86) (end 142.75 86.12) (width 0.5) (layer "F.Cu") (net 19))
 (segment (start 137 81.5) (end 138.25 81.5) (width 0.5) (layer "F.Cu") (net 19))
 (segment (start 138.25 81.5) (end 142.75 86) (width 0.5) (layer "F.Cu") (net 19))
 (segment (start 136.25 82.3125) (end 136.25 82.25) (width 0.5) (layer "F.Cu") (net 19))
 (segment (start 136.25 82.25) (end 137 81.5) (width 0.5) (layer "F.Cu") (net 19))
 (segment (start 122.425 90.575) (end 122.425 92.505) (width 0.5) (layer "F.Cu") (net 17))
 (segment (start 122 85.825) (end 122 87.325) (width 0.5) (layer "F.Cu") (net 17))
 (segment (start 122.425 92.505) (end 122.595 92.675) (width 0.5) (layer "F.Cu") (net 17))
 (segment (start 122.425 87.75) (end 122.425 90.575) (width 0.5) (layer "F.Cu") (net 17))
 (segment (start 117.25 90.51) (end 122.36 90.51) (width 0.5) (layer "F.Cu") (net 17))
 (segment (start 122 87.325) (end 122.425 87.75) (width 0.5) (layer "F.Cu") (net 17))
 (segment (start 122.36 90.51) (end 122.425 90.575) (width 0.5) (layer "F.Cu") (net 17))
 (segment (start 128.8 82.45) (end 128.5 82.75) (width 0.5) (layer "F.Cu") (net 10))
 (segment (start 128.5 82.75) (end 128.5 83.825) (width 0.5) (layer "F.Cu") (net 10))
 (segment (start 128.925 84.25) (end 128.925 84.325) (width 0.5) (layer "F.Cu") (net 10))
 (segment (start 128.5 84.75) (end 128.5 86.175) (width 0.5) (layer "F.Cu") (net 10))
 (segment (start 128.925 84.325) (end 128.5 84.75) (width 0.5) (layer "F.Cu") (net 10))
 (segment (start 128.5 83.825) (end 128.925 84.25) (width 0.5) (layer "F.Cu") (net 10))
 (segment (start 128.8 82.1875) (end 128.8 82.45) (width 0.5) (layer "F.Cu") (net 10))
 (segment (start 135.425 86.25) (end 135.425 86.325) (width 0.5) (layer "F.Cu") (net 12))
 (segment (start 135 87.925) (end 135.25 88.175) (width 0.5) (layer "F.Cu") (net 12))
 (segment (start 135.3 86.125) (end 135.425 86.25) (width 0.5) (layer "F.Cu") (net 12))
 (segment (start 135.3 84.1875) (end 135.3 86.125) (width 0.5) (layer "F.Cu") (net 12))
 (segment (start 135.425 86.325) (end 135 86.75) (width 0.5) (layer "F.Cu") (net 12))
 (segment (start 135 86.75) (end 135 87.925) (width 0.5) (layer "F.Cu") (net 12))
 (segment (start 122.25 82.25) (end 122 82.5) (width 0.5) (layer "F.Cu") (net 7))
 (segment (start 122 82.5) (end 122 84.175) (width 0.5) (layer "F.Cu") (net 7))
 (segment (start 122.05 80.1875) (end 122.05 82.05) (width 0.5) (layer "F.Cu") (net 7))
 (segment (start 122.05 82.05) (end 122.25 82.25) (width 0.5) (layer "F.Cu") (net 7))
 (segment (start 135.25 91.325) (end 135.675 91.75) (width 0.5) (layer "F.Cu") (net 9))
 (segment (start 135.25 90.75) (end 135.25 91.325) (width 0.5) (layer "F.Cu") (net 9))
 (segment (start 135.25 89.825) (end 135.25 90.75) (width 0.5) (layer "F.Cu") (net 9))
 (segment (start 126.405 92.675) (end 133.325 92.675) (width 0.5) (layer "F.Cu") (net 9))
 (segment (start 133.325 92.675) (end 135.25 90.75) (width 0.5) (layer "F.Cu") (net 9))
 (segment (start 128.25 88.25) (end 128.25 89.25) (width 0.5) (layer "F.Cu") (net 11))
 (segment (start 128.75 89.75) (end 128.925 89.75) (width 0.5) (layer "F.Cu") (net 11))
 (segment (start 128.25 89.25) (end 128.75 89.75) (width 0.5) (layer "F.Cu") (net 11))
 (segment (start 125.5 89.75) (end 128.75 89.75) (width 0.5) (layer "F.Cu") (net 11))
 (segment (start 124 91.25) (end 125.5 89.75) (width 0.5) (layer "F.Cu") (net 11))
 (segment (start 123.865 92.675) (end 124 92.54) (width 0.5) (layer "F.Cu") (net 11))
 (segment (start 124 92.54) (end 124 91.25) (width 0.5) (layer "F.Cu") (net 11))
 (segment (start 128.5 87.825) (end 128.5 88) (width 0.5) (layer "F.Cu") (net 11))
 (segment (start 128.5 88) (end 128.25 88.25) (width 0.5) (layer "F.Cu") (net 11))
 (segment (start 122.595 96.655) (end 122.595 97.825) (width 0.5) (layer "F.Cu") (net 13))
 (segment (start 133.925 98) (end 133.25 98) (width 0.5) (layer "F.Cu") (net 13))
 (segment (start 133.25 98) (end 130.75 95.5) (width 0.5) (layer "F.Cu") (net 13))
 (segment (start 130.75 95.5) (end 123.75 95.5) (width 0.5) (layer "F.Cu") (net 13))
 (segment (start 123.75 95.5) (end 122.595 96.655) (width 0.5) (layer "F.Cu") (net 13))
 (segment (start 133.925 95.5) (end 133.925 98) (width 0.5) (layer "F.Cu") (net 13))
 (segment (start 129.75 80.3125) (end 129.75 80) (width 0.5) (layer "F.Cu") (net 20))
 (segment (start 129.75 80) (end 130.5 79.25) (width 0.5) (layer "F.Cu") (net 20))
 (segment (start 137.75 79.25) (end 142.08 83.58) (width 0.5) (layer "F.Cu") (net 20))
 (segment (start 130.5 79.25) (end 137.75 79.25) (width 0.5) (layer "F.Cu") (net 20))
 (segment (start 142.08 83.58) (end 142.75 83.58) (width 0.5) (layer "F.Cu") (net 20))
 (segment (start 141.29 81.04) (end 138.25 78) (width 0.5) (layer "F.Cu") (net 8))
 (segment (start 123.3125 78) (end 123 78.3125) (width 0.5) (layer "F.Cu") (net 8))
 (segment (start 138.25 78) (end 123.3125 78) (width 0.5) (layer "F.Cu") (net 8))
 (segment (start 123 78.25) (end 123 78.3125) (width 0.5) (layer "F.Cu") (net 8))
 (segment (start 142.75 81.04) (end 141.29 81.04) (width 0.5) (layer "F.Cu") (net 8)))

